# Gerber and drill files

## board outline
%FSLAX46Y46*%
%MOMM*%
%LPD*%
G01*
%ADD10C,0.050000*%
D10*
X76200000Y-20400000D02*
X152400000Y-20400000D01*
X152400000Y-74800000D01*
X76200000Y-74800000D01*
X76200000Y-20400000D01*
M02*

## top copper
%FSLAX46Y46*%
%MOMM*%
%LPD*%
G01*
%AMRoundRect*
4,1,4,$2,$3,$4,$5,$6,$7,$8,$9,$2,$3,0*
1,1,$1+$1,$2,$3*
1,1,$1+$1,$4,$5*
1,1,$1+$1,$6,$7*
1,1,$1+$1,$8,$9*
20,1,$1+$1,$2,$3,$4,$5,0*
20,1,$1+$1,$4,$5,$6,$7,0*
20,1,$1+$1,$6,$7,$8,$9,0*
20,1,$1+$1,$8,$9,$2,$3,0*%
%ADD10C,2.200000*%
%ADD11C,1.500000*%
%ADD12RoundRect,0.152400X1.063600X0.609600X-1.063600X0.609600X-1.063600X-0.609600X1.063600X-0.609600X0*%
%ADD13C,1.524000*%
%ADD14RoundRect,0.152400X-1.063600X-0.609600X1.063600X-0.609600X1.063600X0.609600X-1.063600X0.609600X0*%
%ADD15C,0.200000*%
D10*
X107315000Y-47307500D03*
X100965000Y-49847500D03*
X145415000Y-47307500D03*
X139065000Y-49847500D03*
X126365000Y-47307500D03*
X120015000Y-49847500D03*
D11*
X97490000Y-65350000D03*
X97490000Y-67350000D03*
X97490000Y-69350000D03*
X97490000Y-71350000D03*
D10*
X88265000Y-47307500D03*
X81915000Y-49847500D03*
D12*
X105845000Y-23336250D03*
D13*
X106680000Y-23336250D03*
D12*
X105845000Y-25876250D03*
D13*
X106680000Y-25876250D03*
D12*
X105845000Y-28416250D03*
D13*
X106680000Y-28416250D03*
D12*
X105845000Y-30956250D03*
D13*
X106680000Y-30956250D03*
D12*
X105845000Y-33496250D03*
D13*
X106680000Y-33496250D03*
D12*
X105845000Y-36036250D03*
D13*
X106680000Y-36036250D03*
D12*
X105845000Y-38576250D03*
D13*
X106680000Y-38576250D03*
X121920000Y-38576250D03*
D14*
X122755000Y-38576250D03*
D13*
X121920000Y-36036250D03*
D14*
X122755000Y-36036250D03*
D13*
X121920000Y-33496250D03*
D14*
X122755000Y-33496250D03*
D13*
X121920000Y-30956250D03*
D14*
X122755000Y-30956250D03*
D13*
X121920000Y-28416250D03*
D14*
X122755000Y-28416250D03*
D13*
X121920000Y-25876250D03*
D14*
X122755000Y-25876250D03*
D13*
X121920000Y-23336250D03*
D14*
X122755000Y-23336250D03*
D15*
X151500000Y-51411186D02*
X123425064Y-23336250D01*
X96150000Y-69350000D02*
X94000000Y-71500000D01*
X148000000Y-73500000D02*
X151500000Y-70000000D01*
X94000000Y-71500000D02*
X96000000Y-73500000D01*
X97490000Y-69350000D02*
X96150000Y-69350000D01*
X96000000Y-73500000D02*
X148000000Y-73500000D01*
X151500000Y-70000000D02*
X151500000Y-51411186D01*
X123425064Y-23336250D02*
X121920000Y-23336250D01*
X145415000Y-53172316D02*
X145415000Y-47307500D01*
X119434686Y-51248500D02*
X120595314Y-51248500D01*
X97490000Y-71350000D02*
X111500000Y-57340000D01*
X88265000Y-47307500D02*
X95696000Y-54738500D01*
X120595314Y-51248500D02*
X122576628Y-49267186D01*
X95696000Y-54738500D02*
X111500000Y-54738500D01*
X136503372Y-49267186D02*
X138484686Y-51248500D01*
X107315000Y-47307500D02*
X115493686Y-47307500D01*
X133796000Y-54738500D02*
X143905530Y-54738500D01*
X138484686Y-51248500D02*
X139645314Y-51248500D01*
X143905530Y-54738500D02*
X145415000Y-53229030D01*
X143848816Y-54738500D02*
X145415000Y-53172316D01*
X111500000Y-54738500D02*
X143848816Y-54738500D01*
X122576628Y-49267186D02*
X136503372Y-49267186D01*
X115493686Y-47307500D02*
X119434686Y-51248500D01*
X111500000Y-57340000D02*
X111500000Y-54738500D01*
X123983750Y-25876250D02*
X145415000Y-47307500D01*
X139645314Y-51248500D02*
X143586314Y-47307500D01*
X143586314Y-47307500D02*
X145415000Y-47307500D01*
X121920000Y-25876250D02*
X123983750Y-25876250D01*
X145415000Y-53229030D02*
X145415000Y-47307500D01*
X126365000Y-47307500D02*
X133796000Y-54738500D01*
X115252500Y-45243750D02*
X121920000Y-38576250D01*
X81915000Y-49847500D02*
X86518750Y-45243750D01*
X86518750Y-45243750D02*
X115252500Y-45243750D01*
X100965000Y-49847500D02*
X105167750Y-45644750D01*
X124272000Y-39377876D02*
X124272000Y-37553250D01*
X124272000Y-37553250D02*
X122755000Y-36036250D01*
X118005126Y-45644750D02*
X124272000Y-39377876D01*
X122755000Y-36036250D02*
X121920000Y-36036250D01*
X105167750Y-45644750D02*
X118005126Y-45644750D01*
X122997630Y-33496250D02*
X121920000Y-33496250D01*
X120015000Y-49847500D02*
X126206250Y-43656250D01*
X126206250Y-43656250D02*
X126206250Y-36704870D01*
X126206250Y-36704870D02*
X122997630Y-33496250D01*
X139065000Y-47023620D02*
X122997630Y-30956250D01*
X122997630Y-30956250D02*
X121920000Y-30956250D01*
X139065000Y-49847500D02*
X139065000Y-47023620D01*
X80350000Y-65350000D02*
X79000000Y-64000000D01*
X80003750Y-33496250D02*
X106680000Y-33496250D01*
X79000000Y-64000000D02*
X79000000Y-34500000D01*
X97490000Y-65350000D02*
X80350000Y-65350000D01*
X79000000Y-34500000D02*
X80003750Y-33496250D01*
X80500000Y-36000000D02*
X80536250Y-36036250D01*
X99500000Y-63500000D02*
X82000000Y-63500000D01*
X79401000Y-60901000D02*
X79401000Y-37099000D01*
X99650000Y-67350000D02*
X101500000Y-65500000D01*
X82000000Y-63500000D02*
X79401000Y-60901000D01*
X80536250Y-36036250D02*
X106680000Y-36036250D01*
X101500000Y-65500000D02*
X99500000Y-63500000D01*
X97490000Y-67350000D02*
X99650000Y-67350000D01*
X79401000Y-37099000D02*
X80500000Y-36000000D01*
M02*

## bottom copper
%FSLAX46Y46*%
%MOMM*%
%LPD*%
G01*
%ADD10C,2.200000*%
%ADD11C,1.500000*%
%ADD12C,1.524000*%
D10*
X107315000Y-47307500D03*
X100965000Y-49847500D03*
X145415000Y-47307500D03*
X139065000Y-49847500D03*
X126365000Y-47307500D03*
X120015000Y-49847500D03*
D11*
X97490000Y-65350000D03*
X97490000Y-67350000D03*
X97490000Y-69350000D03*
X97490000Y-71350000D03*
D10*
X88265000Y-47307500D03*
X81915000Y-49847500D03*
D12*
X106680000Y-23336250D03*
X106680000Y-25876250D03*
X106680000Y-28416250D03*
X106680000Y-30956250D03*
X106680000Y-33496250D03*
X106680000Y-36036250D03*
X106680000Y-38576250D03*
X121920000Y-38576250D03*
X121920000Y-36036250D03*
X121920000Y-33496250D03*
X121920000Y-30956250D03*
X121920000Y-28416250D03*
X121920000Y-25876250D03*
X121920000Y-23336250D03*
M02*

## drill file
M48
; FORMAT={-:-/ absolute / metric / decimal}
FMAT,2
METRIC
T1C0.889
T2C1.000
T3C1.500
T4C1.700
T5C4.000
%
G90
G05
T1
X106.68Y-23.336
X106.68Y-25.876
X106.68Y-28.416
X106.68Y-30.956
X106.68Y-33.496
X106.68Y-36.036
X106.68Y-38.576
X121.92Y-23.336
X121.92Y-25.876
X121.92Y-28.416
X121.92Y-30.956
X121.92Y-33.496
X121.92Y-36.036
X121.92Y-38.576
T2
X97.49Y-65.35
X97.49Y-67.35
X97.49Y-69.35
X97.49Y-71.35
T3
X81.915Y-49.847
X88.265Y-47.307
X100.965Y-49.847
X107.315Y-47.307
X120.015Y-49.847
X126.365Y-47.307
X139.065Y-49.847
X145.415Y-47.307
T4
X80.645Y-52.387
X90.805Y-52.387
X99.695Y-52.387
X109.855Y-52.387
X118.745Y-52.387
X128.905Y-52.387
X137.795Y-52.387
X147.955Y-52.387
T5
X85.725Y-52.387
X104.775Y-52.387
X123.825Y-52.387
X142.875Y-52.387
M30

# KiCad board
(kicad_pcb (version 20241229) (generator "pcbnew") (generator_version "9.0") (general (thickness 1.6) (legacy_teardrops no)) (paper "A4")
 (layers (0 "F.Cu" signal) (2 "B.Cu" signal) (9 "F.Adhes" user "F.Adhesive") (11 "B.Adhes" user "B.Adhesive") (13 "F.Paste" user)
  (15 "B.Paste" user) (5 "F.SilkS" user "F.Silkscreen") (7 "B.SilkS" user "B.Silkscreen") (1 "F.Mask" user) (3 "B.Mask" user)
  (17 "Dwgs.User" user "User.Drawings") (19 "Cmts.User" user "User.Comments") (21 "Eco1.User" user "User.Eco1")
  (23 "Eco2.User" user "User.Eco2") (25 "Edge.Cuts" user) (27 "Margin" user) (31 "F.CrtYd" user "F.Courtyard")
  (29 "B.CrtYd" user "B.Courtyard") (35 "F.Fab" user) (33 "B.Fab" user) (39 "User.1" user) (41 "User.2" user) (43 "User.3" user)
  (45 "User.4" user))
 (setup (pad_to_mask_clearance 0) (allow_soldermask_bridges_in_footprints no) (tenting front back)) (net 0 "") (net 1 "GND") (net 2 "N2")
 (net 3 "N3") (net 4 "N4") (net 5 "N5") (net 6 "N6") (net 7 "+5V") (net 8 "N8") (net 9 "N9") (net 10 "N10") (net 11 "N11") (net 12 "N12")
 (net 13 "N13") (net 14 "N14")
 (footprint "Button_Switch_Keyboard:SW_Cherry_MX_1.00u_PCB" (layer "F.Cu") (at 107.315 47.3075)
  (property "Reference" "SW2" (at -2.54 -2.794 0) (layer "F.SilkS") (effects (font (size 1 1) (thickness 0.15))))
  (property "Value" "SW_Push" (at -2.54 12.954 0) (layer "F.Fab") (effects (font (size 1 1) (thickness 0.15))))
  (pad "" np_thru_hole circle (at -7.62 5.08) (size 1.7 1.7) (drill 1.7) (layers "*.Cu" "*.Mask"))
  (pad "" np_thru_hole circle (at -2.54 5.08) (size 4 4) (drill 4) (layers "*.Cu" "*.Mask"))
  (pad "" np_thru_hole circle (at 2.54 5.08) (size 1.7 1.7) (drill 1.7) (layers "*.Cu" "*.Mask"))
  (pad "1" thru_hole circle (at 0 0) (size 2.2 2.2) (drill 1.5) (layers "*.Cu" "*.Mask") (remove_unused_layers no) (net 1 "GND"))
  (pad "2" thru_hole circle (at -6.35 2.54) (size 2.2 2.2) (drill 1.5) (layers "*.Cu" "*.Mask") (remove_unused_layers no) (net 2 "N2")))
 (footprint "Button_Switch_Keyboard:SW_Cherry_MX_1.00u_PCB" (layer "F.Cu") (at 145.415 47.3075)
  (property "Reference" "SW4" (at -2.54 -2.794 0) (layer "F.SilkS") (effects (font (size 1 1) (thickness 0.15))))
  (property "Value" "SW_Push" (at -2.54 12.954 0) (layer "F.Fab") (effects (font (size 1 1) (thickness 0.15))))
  (pad "" np_thru_hole circle (at -7.62 5.08) (size 1.7 1.7) (drill 1.7) (layers "*.Cu" "*.Mask"))
  (pad "" np_thru_hole circle (at -2.54 5.08) (size 4 4) (drill 4) (layers "*.Cu" "*.Mask"))
  (pad "" np_thru_hole circle (at 2.54 5.08) (size 1.7 1.7) (drill 1.7) (layers "*.Cu" "*.Mask"))
  (pad "1" thru_hole circle (at 0 0) (size 2.2 2.2) (drill 1.5) (layers "*.Cu" "*.Mask") (remove_unused_layers no) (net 1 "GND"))
  (pad "2" thru_hole circle (at -6.35 2.54) (size 2.2 2.2) (drill 1.5) (layers "*.Cu" "*.Mask") (remove_unused_layers no) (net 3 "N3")))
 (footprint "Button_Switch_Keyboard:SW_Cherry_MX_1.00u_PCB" (layer "F.Cu") (at 126.365 47.3075)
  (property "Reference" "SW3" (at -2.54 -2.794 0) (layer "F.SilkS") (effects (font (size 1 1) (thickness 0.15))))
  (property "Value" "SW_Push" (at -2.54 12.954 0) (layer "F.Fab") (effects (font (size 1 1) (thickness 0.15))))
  (pad "" np_thru_hole circle (at -7.62 5.08) (size 1.7 1.7) (drill 1.7) (layers "*.Cu" "*.Mask"))
  (pad "" np_thru_hole circle (at -2.54 5.08) (size 4 4) (drill 4) (layers "*.Cu" "*.Mask"))
  (pad "" np_thru_hole circle (at 2.54 5.08) (size 1.7 1.7) (drill 1.7) (layers "*.Cu" "*.Mask"))
  (pad "1" thru_hole circle (at 0 0) (size 2.2 2.2) (drill 1.5) (layers "*.Cu" "*.Mask") (remove_unused_layers no) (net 1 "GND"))
  (pad "2" thru_hole circle (at -6.35 2.54) (size 2.2 2.2) (drill 1.5) (layers "*.Cu" "*.Mask") (remove_unused_layers no) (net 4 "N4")))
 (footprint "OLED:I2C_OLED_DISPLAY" (layer "F.Cu") (at 114.24 64.1)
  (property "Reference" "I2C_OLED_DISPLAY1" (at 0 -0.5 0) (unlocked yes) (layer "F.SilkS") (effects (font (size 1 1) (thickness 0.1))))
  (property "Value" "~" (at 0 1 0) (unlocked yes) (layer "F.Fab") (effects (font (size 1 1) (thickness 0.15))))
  (pad "1" thru_hole circle (at -16.75 1.25 90) (size 1.5 1.5) (drill 1) (layers "*.Cu" "*.Mask") (remove_unused_layers no) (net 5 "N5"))
  (pad "2" thru_hole circle (at -16.75 3.25 90) (size 1.5 1.5) (drill 1) (layers "*.Cu" "*.Mask") (remove_unused_layers no) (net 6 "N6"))
  (pad "3" thru_hole circle (at -16.75 5.25 90) (size 1.5 1.5) (drill 1) (layers "*.Cu" "*.Mask") (remove_unused_layers no) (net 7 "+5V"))
  (pad "4" thru_hole circle (at -16.75 7.25 90) (size 1.5 1.5) (drill 1) (layers "*.Cu" "*.Mask") (remove_unused_layers no) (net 1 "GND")))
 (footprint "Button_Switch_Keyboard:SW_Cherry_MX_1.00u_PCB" (layer "F.Cu") (at 88.265 47.3075)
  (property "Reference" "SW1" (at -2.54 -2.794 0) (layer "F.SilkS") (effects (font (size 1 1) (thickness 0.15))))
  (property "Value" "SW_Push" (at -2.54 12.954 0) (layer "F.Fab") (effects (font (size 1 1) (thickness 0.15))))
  (pad "" np_thru_hole circle (at -7.62 5.08) (size 1.7 1.7) (drill 1.7) (layers "*.Cu" "*.Mask"))
  (pad "" np_thru_hole circle (at -2.54 5.08) (size 4 4) (drill 4) (layers "*.Cu" "*.Mask"))
  (pad "" np_thru_hole circle (at 2.54 5.08) (size 1.7 1.7) (drill 1.7) (layers "*.Cu" "*.Mask"))
  (pad "1" thru_hole circle (at 0 0) (size 2.2 2.2) (drill 1.5) (layers "*.Cu" "*.Mask") (remove_unused_layers no) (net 1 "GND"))
  (pad "2" thru_hole circle (at -6.35 2.54) (size 2.2 2.2) (drill 1.5) (layers "*.Cu" "*.Mask") (remove_unused_layers no) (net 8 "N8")))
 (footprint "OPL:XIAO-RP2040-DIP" (layer "F.Cu") (at 114.3 30.95625)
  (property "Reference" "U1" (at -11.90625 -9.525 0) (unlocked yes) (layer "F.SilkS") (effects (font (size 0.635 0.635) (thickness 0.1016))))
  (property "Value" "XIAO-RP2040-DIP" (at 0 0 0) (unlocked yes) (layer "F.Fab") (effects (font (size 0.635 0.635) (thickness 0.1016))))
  (pad "1" smd roundrect (at -8.455 -7.62 180) (size 2.432 1.524) (layers "F.Cu" "F.Mask") (roundrect_rratio 0.1) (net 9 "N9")
   (thermal_bridge_angle 45))
  (pad "1" thru_hole circle (at -7.62 -7.62 180) (size 1.524 1.524) (drill 0.889) (layers "*.Cu" "*.Mask") (remove_unused_layers no)
   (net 9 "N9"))
  (pad "2" smd roundrect (at -8.455 -5.08 180) (size 2.432 1.524) (layers "F.Cu" "F.Mask") (roundrect_rratio 0.1) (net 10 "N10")
   (thermal_bridge_angle 45))
  (pad "2" thru_hole circle (at -7.62 -5.08 180) (size 1.524 1.524) (drill 0.889) (layers "*.Cu" "*.Mask") (remove_unused_layers no)
   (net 10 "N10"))
  (pad "3" smd roundrect (at -8.455 -2.54 180) (size 2.432 1.524) (layers "F.Cu" "F.Mask") (roundrect_rratio 0.1) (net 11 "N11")
   (thermal_bridge_angle 45))
  (pad "3" thru_hole circle (at -7.62 -2.54 180) (size 1.524 1.524) (drill 0.889) (layers "*.Cu" "*.Mask") (remove_unused_layers no)
   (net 11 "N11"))
  (pad "4" smd roundrect (at -8.455 0 180) (size 2.432 1.524) (layers "F.Cu" "F.Mask") (roundrect_rratio 0.1) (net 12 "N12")
   (thermal_bridge_angle 45))
  (pad "4" thru_hole circle (at -7.62 0 180) (size 1.524 1.524) (drill 0.889) (layers "*.Cu" "*.Mask") (remove_unused_layers no)
   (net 12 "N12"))
  (pad "5" smd roundrect (at -8.455 2.54 180) (size 2.432 1.524) (layers "F.Cu" "F.Mask") (roundrect_rratio 0.1) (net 5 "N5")
   (thermal_bridge_angle 45))
  (pad "5" thru_hole circle (at -7.62 2.54 180) (size 1.524 1.524) (drill 0.889) (layers "*.Cu" "*.Mask") (remove_unused_layers no)
   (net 5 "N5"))
  (pad "6" smd roundrect (at -8.455 5.08 180) (size 2.432 1.524) (layers "F.Cu" "F.Mask") (roundrect_rratio 0.1) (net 6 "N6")
   (thermal_bridge_angle 45))
  (pad "6" thru_hole circle (at -7.62 5.08 180) (size 1.524 1.524) (drill 0.889) (layers "*.Cu" "*.Mask") (remove_unused_layers no)
   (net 6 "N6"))
  (pad "7" smd roundrect (at -8.455 7.62 180) (size 2.432 1.524) (layers "F.Cu" "F.Mask") (roundrect_rratio 0.1) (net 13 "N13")
   (thermal_bridge_angle 45))
  (pad "7" thru_hole circle (at -7.62 7.62 180) (size 1.524 1.524) (drill 0.889) (layers "*.Cu" "*.Mask") (remove_unused_layers no)
   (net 13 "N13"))
  (pad "8" thru_hole circle (at 7.62 7.62) (size 1.524 1.524) (drill 0.889) (layers "*.Cu" "*.Mask") (remove_unused_layers no) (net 8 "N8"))
  (pad "8" smd roundrect (at 8.455 7.62) (size 2.432 1.524) (layers "F.Cu" "F.Mask") (roundrect_rratio 0.1) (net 8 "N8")
   (thermal_bridge_angle 45))
  (pad "9" thru_hole circle (at 7.62 5.08) (size 1.524 1.524) (drill 0.889) (layers "*.Cu" "*.Mask") (remove_unused_layers no) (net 2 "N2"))
  (pad "9" smd roundrect (at 8.455 5.08) (size 2.432 1.524) (layers "F.Cu" "F.Mask") (roundrect_rratio 0.1) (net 2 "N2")
   (thermal_bridge_angle 45))
  (pad "10" thru_hole circle (at 7.62 2.54) (size 1.524 1.524) (drill 0.889) (layers "*.Cu" "*.Mask") (remove_unused_layers no) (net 4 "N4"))
  (pad "10" smd roundrect (at 8.455 2.54) (size 2.432 1.524) (layers "F.Cu" "F.Mask") (roundrect_rratio 0.1) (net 4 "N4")
   (thermal_bridge_angle 45))
  (pad "11" thru_hole circle (at 7.62 0) (size 1.524 1.524) (drill 0.889) (layers "*.Cu" "*.Mask") (remove_unused_layers no) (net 3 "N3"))
  (pad "11" smd roundrect (at 8.455 0) (size 2.432 1.524) (layers "F.Cu" "F.Mask") (roundrect_rratio 0.1) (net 3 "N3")
   (thermal_bridge_angle 45))
  (pad "12" thru_hole circle (at 7.62 -2.54) (size 1.524 1.524) (drill 0.889) (layers "*.Cu" "*.Mask") (remove_unused_layers no)
   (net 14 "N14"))
  (pad "12" smd roundrect (at 8.455 -2.54) (size 2.432 1.524) (layers "F.Cu" "F.Mask") (roundrect_rratio 0.1) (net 14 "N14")
   (thermal_bridge_angle 45))
  (pad "13" thru_hole circle (at 7.62 -5.08) (size 1.524 1.524) (drill 0.889) (layers "*.Cu" "*.Mask") (remove_unused_layers no)
   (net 1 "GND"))
  (pad "13" smd roundrect (at 8.455 -5.08) (size 2.432 1.524) (layers "F.Cu" "F.Mask") (roundrect_rratio 0.1) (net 1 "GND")
   (thermal_bridge_angle 45))
  (pad "14" thru_hole circle (at 7.62 -7.62) (size 1.524 1.524) (drill 0.889) (layers "*.Cu" "*.Mask") (remove_unused_layers no)
   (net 7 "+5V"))
  (pad "14" smd roundrect (at 8.455 -7.62) (size 2.432 1.524) (layers "F.Cu" "F.Mask") (roundrect_rratio 0.1) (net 7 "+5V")
   (thermal_bridge_angle 45)))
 (gr_rect (start 76.2 20.4) (end 152.4 74.8) (stroke (width 0.05) (type default)) (fill no) (layer "Edge.Cuts"))
 (segment (start 151.5 51.411186) (end 123.425064 23.33625) (width 0.2) (layer "F.Cu") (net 7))
 (segment (start 96.15 69.35) (end 94 71.5) (width 0.2) (layer "F.Cu") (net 7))
 (segment (start 148 73.5) (end 151.5 70) (width 0.2) (layer "F.Cu") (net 7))
 (segment (start 94 71.5) (end 96 73.5) (width 0.2) (layer "F.Cu") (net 7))
 (segment (start 97.49 69.35) (end 96.15 69.35) (width 0.2) (layer "F.Cu") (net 7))
 (segment (start 96 73.5) (end 148 73.5) (width 0.2) (layer "F.Cu") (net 7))
 (segment (start 151.5 70) (end 151.5 51.411186) (width 0.2) (layer "F.Cu") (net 7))
 (segment (start 123.425064 23.33625) (end 121.92 23.33625) (width 0.2) (layer "F.Cu") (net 7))
 (segment (start 145.415 53.172316) (end 145.415 47.3075) (width 0.2) (layer "F.Cu") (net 1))
 (segment (start 119.434686 51.2485) (end 120.595314 51.2485) (width 0.2) (layer "F.Cu") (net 1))
 (segment (start 97.49 71.35) (end 111.5 57.34) (width 0.2) (layer "F.Cu") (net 1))
 (segment (start 88.265 47.3075) (end 95.696 54.7385) (width 0.2) (layer "F.Cu") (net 1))
 (segment (start 120.595314 51.2485) (end 122.576628 49.267186) (width 0.2) (layer "F.Cu") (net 1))
 (segment (start 95.696 54.7385) (end 111.5 54.7385) (width 0.2) (layer "F.Cu") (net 1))
 (segment (start 136.503372 49.267186) (end 138.484686 51.2485) (width 0.2) (layer "F.Cu") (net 1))
 (segment (start 107.315 47.3075) (end 115.493686 47.3075) (width 0.2) (layer "F.Cu") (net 1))
 (segment (start 133.796 54.7385) (end 143.90553 54.7385) (width 0.2) (layer "F.Cu") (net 1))
 (segment (start 138.484686 51.2485) (end 139.645314 51.2485) (width 0.2) (layer "F.Cu") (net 1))
 (segment (start 143.90553 54.7385) (end 145.415 53.22903) (width 0.2) (layer "F.Cu") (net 1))
 (segment (start 143.848816 54.7385) (end 145.415 53.172316) (width 0.2) (layer "F.Cu") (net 1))
 (segment (start 111.5 54.7385) (end 143.848816 54.7385) (width 0.2) (layer "F.Cu") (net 1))
 (segment (start 122.576628 49.267186) (end 136.503372 49.267186) (width 0.2) (layer "F.Cu") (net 1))
 (segment (start 115.493686 47.3075) (end 119.434686 51.2485) (width 0.2) (layer "F.Cu") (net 1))
 (segment (start 111.5 57.34) (end 111.5 54.7385) (width 0.2) (layer "F.Cu") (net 1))
 (segment (start 123.98375 25.87625) (end 145.415 47.3075) (width 0.2) (layer "F.Cu") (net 1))
 (segment (start 139.645314 51.2485) (end 143.586314 47.3075) (width 0.2) (layer "F.Cu") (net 1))
 (segment (start 143.586314 47.3075) (end 145.415 47.3075) (width 0.2) (layer "F.Cu") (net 1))
 (segment (start 121.92 25.87625) (end 123.98375 25.87625) (width 0.2) (layer "F.Cu") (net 1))
 (segment (start 145.415 53.22903) (end 145.415 47.3075) (width 0.2) (layer "F.Cu") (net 1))
 (segment (start 126.365 47.3075) (end 133.796 54.7385) (width 0.2) (layer "F.Cu") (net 1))
 (segment (start 115.2525 45.24375) (end 121.92 38.57625) (width 0.2) (layer "F.Cu") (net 8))
 (segment (start 81.915 49.8475) (end 86.51875 45.24375) (width 0.2) (layer "F.Cu") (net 8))
 (segment (start 86.51875 45.24375) (end 115.2525 45.24375) (width 0.2) (layer "F.Cu") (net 8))
 (segment (start 100.965 49.8475) (end 105.16775 45.64475) (width 0.2) (layer "F.Cu") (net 2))
 (segment (start 124.272 39.377876) (end 124.272 37.55325) (width 0.2) (layer "F.Cu") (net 2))
 (segment (start 124.272 37.55325) (end 122.755 36.03625) (width 0.2) (layer "F.Cu") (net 2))
 (segment (start 118.005126 45.64475) (end 124.272 39.377876) (width 0.2) (layer "F.Cu") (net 2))
 (segment (start 122.755 36.03625) (end 121.92 36.03625) (width 0.2) (layer "F.Cu") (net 2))
 (segment (start 105.16775 45.64475) (end 118.005126 45.64475) (width 0.2) (layer "F.Cu") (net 2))
 (segment (start 122.99763 33.49625) (end 121.92 33.49625) (width 0.2) (layer "F.Cu") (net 4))
 (segment (start 120.015 49.8475) (end 126.20625 43.65625) (width 0.2) (layer "F.Cu") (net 4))
 (segment (start 126.20625 43.65625) (end 126.20625 36.70487) (width 0.2) (layer "F.Cu") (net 4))
 (segment (start 126.20625 36.70487) (end 122.99763 33.49625) (width 0.2) (layer "F.Cu") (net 4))
 (segment (start 139.065 47.02362) (end 122.99763 30.95625) (width 0.2) (layer "F.Cu") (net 3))
 (segment (start 122.99763 30.95625) (end 121.92 30.95625) (width 0.2) (layer "F.Cu") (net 3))
 (segment (start 139.065 49.8475) (end 139.065 47.02362) (width 0.2) (layer "F.Cu") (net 3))
 (segment (start 80.35 65.35) (end 79 64) (width 0.2) (layer "F.Cu") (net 5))
 (segment (start 80.00375 33.49625) (end 106.68 33.49625) (width 0.2) (layer "F.Cu") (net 5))
 (segment (start 79 64) (end 79 34.5) (width 0.2) (layer "F.Cu") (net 5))
 (segment (start 97.49 65.35) (end 80.35 65.35) (width 0.2) (layer "F.Cu") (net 5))
 (segment (start 79 34.5) (end 80.00375 33.49625) (width 0.2) (layer "F.Cu") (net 5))
 (segment (start 80.5 36) (end 80.53625 36.03625) (width 0.2) (layer "F.Cu") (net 6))
 (segment (start 99.5 63.5) (end 82 63.5) (width 0.2) (layer "F.Cu") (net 6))
 (segment (start 79.401 60.901) (end 79.401 37.099) (width 0.2) (layer "F.Cu") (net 6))
 (segment (start 99.65 67.35) (end 101.5 65.5) (width 0.2) (layer "F.Cu") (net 6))
 (segment (start 82 63.5) (end 79.401 60.901) (width 0.2) (layer "F.Cu") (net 6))
 (segment (start 80.53625 36.03625) (end 106.68 36.03625) (width 0.2) (layer "F.Cu") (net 6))
 (segment (start 101.5 65.5) (end 99.5 63.5) (width 0.2) (layer "F.Cu") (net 6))
 (segment (start 97.49 67.35) (end 99.65 67.35) (width 0.2) (layer "F.Cu") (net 6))
 (segment (start 79.401 37.099) (end 80.5 36) (width 0.2) (layer "F.Cu") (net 6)))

